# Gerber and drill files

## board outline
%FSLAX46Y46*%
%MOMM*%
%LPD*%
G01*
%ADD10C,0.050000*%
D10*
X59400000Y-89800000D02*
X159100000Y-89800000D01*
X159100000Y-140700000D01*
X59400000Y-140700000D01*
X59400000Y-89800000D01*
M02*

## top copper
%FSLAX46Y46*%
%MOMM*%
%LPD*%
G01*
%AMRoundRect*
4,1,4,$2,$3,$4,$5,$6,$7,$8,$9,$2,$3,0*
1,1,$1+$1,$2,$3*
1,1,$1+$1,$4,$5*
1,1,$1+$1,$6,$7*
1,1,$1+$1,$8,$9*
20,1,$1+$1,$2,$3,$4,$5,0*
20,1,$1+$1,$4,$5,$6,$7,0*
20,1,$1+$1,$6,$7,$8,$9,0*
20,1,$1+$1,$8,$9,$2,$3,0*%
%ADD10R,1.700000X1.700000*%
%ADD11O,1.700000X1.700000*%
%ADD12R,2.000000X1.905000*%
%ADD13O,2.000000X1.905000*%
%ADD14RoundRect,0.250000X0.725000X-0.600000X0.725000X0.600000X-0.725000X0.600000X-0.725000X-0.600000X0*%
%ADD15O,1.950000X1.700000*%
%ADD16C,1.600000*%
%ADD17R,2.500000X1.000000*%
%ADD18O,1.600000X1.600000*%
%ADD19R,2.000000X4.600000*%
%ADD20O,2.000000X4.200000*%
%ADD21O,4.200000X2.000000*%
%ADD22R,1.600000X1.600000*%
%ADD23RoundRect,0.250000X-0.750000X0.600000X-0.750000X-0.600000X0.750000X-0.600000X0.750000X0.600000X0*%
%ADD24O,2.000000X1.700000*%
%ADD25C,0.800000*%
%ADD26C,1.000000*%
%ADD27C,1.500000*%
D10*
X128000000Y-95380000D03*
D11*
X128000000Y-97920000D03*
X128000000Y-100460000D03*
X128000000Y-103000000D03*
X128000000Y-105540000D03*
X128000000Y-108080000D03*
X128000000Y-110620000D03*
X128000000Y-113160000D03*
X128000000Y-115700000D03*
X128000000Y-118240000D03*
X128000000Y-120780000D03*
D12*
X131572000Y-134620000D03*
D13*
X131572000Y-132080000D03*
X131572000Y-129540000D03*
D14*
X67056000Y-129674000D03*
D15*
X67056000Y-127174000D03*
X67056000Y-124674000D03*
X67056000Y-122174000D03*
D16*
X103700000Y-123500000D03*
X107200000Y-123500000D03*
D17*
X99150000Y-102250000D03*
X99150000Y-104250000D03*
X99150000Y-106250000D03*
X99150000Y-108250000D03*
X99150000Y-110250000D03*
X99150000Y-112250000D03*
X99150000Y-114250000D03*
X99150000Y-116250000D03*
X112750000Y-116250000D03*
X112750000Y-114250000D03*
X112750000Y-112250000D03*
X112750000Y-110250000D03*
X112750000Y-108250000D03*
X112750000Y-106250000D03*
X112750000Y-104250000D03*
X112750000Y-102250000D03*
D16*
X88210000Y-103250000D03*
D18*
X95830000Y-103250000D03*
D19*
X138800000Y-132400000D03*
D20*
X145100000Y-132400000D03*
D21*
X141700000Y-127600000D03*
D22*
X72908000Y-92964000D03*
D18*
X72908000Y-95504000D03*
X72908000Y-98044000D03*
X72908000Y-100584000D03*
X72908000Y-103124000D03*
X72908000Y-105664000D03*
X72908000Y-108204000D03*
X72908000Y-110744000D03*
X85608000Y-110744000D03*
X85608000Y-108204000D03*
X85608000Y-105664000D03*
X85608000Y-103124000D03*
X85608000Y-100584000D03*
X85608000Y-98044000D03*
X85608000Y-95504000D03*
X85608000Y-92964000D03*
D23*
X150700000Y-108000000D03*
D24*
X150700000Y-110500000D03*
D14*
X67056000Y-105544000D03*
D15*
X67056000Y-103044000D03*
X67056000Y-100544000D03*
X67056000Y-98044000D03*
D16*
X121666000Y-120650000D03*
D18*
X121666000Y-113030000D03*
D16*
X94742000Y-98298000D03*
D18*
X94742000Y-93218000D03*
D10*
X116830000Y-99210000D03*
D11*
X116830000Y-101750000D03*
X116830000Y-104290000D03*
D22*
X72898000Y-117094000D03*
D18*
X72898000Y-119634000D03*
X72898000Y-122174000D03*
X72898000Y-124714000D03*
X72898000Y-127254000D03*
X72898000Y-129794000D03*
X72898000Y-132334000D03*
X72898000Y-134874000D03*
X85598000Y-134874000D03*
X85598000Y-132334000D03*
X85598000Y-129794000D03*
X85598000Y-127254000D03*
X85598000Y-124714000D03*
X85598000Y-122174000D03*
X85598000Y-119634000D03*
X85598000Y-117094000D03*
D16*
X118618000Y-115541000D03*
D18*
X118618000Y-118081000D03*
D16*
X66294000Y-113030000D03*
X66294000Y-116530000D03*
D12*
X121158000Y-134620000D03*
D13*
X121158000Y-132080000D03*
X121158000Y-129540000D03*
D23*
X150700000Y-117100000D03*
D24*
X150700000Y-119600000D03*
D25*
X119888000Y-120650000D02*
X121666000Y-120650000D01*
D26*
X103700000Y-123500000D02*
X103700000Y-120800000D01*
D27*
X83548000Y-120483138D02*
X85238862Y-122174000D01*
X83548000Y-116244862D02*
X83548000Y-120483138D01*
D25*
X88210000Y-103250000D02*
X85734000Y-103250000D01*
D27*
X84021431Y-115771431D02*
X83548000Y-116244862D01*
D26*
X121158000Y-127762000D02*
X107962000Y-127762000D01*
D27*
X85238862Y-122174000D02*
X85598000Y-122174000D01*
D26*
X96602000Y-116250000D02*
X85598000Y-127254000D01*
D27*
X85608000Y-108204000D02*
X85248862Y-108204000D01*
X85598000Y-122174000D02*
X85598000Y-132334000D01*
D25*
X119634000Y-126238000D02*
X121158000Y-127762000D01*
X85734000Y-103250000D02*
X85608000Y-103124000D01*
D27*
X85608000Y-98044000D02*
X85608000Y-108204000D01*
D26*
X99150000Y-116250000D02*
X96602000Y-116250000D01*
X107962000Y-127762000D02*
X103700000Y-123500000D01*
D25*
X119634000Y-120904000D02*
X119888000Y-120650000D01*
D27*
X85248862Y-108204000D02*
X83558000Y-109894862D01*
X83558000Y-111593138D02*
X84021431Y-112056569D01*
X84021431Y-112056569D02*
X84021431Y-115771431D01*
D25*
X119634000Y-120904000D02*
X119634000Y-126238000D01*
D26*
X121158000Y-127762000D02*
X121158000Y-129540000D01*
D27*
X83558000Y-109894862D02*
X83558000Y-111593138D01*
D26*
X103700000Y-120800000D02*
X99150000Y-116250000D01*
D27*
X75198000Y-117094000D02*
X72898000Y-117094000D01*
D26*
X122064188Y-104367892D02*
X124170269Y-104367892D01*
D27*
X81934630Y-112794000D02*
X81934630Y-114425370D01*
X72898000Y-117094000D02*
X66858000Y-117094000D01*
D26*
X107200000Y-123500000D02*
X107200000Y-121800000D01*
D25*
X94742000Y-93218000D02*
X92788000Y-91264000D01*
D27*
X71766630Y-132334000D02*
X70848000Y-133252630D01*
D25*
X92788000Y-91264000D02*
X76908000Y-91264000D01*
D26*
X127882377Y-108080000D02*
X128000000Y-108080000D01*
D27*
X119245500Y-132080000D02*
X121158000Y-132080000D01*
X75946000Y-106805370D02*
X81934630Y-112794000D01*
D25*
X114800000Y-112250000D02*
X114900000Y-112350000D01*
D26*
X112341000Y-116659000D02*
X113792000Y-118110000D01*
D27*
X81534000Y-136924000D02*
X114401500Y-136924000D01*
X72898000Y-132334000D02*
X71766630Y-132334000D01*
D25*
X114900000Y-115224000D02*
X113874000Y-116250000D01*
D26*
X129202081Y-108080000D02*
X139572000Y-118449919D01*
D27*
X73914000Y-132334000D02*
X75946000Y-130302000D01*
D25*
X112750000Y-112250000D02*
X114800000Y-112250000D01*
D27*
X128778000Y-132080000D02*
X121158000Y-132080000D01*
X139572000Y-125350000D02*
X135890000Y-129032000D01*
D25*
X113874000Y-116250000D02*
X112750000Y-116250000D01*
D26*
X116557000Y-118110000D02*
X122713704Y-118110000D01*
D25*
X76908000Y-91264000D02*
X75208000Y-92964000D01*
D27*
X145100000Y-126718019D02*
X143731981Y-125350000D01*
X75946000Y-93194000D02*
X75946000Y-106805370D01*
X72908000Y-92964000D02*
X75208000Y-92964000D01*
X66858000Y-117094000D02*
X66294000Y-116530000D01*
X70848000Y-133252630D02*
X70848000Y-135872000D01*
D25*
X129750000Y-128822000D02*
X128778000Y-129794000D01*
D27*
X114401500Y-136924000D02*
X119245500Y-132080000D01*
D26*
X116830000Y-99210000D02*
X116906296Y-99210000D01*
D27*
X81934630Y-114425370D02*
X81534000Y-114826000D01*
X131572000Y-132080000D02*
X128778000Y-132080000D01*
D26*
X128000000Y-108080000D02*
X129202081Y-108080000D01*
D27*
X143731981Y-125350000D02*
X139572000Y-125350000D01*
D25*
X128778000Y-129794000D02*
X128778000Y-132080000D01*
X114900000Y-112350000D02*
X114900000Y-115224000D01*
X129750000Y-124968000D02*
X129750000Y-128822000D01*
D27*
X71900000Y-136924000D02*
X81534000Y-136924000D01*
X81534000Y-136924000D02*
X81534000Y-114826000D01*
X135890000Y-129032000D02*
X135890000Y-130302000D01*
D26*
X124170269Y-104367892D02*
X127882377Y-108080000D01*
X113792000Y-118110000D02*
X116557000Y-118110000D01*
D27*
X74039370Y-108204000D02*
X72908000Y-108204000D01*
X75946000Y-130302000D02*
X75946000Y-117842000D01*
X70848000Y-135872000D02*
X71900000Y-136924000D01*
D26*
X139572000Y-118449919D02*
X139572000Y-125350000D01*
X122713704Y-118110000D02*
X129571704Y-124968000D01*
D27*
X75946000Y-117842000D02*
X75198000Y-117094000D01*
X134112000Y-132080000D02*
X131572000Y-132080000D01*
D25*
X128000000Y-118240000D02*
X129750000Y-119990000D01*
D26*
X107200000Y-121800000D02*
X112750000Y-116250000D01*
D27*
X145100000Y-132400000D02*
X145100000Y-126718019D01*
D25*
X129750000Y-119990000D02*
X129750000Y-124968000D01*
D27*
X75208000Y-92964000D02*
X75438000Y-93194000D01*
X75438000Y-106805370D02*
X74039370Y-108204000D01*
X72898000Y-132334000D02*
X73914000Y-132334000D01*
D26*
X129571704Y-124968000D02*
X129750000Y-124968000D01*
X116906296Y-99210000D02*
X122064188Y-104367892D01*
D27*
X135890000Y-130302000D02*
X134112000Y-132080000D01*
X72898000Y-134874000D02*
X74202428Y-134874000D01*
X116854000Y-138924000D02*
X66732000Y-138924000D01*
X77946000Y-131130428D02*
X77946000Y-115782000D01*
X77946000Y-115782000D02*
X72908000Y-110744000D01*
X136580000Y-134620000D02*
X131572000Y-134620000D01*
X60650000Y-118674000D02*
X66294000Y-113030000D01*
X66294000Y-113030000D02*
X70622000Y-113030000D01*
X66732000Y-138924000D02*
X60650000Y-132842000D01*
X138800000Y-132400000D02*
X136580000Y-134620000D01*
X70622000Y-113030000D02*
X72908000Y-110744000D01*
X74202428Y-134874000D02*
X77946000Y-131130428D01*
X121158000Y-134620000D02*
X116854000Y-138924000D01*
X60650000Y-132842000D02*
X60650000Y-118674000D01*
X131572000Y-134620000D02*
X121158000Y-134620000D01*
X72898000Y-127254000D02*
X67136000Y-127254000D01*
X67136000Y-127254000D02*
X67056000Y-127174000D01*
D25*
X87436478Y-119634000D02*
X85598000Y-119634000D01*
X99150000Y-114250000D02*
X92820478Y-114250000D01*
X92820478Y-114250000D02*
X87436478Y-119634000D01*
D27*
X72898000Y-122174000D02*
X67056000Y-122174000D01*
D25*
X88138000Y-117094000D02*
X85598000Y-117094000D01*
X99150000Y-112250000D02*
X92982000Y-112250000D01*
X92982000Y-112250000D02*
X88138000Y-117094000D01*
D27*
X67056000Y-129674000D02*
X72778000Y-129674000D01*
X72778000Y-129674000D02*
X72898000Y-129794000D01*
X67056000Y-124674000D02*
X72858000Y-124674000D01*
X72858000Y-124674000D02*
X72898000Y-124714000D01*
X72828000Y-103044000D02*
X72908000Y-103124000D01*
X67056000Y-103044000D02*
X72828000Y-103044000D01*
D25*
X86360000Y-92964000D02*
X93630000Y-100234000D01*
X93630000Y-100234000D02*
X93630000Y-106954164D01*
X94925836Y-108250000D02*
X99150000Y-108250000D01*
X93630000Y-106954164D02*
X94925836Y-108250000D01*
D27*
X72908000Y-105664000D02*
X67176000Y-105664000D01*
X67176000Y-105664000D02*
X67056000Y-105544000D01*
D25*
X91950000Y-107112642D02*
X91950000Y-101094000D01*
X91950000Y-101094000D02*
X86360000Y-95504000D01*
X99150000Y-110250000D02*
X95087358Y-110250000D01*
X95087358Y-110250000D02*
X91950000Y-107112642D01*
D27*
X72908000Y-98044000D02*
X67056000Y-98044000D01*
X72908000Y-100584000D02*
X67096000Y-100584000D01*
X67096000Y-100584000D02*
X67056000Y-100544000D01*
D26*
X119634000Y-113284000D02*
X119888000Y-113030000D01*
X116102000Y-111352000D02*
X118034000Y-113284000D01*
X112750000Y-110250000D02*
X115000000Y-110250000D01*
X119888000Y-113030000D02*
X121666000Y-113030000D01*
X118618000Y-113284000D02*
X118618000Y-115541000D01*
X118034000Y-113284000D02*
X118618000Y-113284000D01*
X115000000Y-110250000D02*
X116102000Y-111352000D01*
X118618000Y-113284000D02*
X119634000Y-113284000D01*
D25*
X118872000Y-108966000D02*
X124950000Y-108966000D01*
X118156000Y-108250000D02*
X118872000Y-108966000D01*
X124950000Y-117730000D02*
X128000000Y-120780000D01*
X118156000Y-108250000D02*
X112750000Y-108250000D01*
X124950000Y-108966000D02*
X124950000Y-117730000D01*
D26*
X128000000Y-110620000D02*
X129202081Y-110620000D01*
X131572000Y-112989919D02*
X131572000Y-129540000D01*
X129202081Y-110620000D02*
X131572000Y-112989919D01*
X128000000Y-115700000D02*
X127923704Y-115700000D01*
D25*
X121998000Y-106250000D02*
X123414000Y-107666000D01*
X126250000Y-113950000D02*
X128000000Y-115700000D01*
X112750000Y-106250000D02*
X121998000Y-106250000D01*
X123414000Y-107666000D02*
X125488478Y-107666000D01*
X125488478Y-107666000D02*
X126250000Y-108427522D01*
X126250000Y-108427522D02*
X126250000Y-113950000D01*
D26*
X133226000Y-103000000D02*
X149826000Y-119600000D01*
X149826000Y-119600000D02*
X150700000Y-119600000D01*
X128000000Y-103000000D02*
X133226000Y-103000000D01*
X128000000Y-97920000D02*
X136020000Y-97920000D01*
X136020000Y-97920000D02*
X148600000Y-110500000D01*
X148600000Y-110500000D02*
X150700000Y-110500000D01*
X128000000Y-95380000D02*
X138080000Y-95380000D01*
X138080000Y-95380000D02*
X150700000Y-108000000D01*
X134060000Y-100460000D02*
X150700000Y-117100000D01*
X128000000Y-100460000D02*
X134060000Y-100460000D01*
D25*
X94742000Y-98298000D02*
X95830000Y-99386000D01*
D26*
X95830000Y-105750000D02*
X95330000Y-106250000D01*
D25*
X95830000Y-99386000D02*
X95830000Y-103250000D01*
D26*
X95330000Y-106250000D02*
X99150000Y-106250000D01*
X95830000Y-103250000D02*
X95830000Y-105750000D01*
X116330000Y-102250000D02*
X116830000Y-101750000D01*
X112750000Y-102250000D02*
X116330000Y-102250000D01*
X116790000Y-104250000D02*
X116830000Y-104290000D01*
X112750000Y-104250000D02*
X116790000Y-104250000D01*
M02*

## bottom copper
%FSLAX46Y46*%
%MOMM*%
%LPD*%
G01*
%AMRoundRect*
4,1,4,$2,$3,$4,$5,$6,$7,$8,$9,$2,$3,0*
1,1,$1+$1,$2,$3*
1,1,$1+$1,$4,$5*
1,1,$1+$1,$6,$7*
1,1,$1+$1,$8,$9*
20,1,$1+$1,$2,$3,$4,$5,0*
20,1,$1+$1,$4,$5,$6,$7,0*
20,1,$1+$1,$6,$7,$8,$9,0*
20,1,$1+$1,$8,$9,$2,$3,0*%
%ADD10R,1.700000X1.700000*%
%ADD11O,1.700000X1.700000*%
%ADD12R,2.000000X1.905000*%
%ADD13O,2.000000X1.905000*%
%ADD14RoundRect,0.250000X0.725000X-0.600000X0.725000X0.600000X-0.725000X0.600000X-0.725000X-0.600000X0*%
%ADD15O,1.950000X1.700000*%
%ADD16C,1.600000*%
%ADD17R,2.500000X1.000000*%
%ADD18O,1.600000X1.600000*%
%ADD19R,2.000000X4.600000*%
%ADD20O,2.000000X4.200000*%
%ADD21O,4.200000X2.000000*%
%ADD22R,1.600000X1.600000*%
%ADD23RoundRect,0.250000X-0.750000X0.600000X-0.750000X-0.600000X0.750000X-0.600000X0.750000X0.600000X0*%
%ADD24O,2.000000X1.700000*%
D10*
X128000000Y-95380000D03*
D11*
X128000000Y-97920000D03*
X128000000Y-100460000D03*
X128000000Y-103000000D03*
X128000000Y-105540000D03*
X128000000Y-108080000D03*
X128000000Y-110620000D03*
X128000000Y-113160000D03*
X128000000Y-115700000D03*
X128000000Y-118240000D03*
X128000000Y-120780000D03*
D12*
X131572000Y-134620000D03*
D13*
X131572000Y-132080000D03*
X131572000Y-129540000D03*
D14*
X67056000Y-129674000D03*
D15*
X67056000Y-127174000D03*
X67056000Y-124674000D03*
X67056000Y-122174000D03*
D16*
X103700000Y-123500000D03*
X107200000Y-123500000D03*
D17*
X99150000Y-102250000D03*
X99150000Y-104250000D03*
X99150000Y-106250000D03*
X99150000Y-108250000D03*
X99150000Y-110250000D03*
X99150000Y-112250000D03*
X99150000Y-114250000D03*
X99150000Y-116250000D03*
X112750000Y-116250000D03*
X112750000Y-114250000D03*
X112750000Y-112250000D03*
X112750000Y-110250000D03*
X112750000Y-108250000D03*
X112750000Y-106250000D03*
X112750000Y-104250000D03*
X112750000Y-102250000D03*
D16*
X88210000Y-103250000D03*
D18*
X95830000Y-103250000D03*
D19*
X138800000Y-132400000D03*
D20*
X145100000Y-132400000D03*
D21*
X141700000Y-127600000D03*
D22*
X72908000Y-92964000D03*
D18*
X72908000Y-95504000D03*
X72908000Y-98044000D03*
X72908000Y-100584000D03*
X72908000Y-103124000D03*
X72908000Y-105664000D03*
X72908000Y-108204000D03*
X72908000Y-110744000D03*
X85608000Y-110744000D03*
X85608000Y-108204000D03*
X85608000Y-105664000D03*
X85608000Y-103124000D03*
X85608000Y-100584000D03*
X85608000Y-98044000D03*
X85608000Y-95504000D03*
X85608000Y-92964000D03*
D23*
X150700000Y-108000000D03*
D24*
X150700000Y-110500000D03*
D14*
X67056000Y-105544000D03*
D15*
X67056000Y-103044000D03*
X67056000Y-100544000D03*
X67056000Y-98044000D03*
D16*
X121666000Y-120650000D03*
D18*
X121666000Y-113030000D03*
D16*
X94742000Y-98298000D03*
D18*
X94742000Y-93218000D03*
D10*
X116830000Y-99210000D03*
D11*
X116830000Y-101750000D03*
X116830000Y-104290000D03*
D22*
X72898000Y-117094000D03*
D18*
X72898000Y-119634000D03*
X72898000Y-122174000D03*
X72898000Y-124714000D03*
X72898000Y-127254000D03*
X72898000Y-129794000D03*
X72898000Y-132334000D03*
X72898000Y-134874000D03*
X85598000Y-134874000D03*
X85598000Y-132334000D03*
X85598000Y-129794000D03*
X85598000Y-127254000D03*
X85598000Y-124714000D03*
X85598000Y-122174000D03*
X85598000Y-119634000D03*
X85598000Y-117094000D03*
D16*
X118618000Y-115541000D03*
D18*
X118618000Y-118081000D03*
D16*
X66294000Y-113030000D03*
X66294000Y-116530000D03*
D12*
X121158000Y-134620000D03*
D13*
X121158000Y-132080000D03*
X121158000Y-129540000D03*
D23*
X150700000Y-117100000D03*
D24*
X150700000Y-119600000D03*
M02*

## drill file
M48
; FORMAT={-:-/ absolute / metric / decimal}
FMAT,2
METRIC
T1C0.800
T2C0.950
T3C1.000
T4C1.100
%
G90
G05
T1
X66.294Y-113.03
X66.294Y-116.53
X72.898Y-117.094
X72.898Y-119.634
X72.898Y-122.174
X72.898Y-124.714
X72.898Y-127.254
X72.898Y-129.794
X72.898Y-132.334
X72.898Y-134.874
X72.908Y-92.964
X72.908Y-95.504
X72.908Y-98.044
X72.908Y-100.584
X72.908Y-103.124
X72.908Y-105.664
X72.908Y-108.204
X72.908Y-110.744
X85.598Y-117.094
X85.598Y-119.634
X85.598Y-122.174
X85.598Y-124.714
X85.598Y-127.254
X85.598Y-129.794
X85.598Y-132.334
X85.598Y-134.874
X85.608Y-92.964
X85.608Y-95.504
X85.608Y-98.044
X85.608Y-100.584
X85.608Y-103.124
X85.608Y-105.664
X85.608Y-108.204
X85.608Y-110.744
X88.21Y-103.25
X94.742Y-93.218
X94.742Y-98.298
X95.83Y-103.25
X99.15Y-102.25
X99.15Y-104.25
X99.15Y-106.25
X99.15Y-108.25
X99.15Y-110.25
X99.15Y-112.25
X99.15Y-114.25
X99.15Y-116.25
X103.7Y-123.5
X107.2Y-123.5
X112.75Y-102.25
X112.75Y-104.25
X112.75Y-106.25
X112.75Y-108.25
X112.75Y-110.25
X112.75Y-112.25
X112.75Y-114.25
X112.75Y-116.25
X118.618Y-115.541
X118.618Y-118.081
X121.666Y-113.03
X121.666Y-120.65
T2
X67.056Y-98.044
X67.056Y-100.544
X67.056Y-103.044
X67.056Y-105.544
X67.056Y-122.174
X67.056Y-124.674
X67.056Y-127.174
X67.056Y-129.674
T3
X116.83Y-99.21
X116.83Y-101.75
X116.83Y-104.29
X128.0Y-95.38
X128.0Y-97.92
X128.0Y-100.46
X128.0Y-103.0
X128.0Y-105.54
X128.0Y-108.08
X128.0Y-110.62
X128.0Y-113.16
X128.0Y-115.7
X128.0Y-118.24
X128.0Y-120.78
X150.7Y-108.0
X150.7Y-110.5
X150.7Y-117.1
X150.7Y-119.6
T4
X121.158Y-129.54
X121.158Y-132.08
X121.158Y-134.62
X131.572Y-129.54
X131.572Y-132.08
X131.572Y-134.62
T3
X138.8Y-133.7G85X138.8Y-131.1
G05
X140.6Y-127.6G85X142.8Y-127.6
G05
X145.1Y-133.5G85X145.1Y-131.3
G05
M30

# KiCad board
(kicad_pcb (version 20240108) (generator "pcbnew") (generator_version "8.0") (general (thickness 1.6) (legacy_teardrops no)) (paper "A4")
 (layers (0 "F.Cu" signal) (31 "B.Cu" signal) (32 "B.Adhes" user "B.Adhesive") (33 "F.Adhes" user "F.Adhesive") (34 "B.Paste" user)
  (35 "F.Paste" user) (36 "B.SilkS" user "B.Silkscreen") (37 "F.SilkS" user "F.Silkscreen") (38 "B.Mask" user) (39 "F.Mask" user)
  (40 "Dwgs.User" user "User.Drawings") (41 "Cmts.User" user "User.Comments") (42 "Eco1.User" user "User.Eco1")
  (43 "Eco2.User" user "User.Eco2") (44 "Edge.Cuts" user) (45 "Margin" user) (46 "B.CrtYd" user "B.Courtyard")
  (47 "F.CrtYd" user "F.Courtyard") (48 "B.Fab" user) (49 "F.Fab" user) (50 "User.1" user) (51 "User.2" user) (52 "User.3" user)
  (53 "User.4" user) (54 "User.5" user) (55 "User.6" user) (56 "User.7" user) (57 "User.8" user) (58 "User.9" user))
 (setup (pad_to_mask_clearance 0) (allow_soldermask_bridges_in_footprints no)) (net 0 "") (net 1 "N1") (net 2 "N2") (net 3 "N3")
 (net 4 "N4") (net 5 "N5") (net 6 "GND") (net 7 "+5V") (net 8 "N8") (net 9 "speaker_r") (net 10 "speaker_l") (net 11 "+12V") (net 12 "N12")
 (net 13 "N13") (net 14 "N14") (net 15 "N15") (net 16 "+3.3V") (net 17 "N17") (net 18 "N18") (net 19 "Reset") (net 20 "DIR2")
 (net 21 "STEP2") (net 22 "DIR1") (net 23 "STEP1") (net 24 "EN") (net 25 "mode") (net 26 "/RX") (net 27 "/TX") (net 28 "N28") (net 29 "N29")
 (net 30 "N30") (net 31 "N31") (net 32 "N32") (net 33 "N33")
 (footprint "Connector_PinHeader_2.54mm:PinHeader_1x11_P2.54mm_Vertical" (layer "F.Cu") (at 128 95.38)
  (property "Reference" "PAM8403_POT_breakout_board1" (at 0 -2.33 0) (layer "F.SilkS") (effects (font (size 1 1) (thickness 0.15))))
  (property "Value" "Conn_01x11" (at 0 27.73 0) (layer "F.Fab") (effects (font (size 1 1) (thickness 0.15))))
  (pad "1" thru_hole rect (at 0 0) (size 1.7 1.7) (drill 1) (layers "*.Cu" "*.Mask") (remove_unused_layers no) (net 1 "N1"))
  (pad "2" thru_hole oval (at 0 2.54) (size 1.7 1.7) (drill 1) (layers "*.Cu" "*.Mask") (remove_unused_layers no) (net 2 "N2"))
  (pad "3" thru_hole oval (at 0 5.08) (size 1.7 1.7) (drill 1) (layers "*.Cu" "*.Mask") (remove_unused_layers no) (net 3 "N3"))
  (pad "4" thru_hole oval (at 0 7.62) (size 1.7 1.7) (drill 1) (layers "*.Cu" "*.Mask") (remove_unused_layers no) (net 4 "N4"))
  (pad "5" thru_hole oval (at 0 10.16) (size 1.7 1.7) (drill 1) (layers "*.Cu" "*.Mask") (remove_unused_layers no) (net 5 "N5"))
  (pad "6" thru_hole oval (at 0 12.7) (size 1.7 1.7) (drill 1) (layers "*.Cu" "*.Mask") (remove_unused_layers no) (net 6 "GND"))
  (pad "7" thru_hole oval (at 0 15.24) (size 1.7 1.7) (drill 1) (layers "*.Cu" "*.Mask") (remove_unused_layers no) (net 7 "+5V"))
  (pad "8" thru_hole oval (at 0 17.78) (size 1.7 1.7) (drill 1) (layers "*.Cu" "*.Mask") (remove_unused_layers no) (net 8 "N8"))
  (pad "9" thru_hole oval (at 0 20.32) (size 1.7 1.7) (drill 1) (layers "*.Cu" "*.Mask") (remove_unused_layers no) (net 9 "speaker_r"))
  (pad "10" thru_hole oval (at 0 22.86) (size 1.7 1.7) (drill 1) (layers "*.Cu" "*.Mask") (remove_unused_layers no) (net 6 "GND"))
  (pad "11" thru_hole oval (at 0 25.4) (size 1.7 1.7) (drill 1) (layers "*.Cu" "*.Mask") (remove_unused_layers no) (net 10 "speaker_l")))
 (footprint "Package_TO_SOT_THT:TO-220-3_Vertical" (layer "F.Cu") (at 131.572 134.62 90)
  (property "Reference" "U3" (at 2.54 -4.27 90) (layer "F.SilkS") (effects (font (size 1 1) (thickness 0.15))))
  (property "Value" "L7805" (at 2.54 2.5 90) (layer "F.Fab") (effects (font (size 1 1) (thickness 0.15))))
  (pad "1" thru_hole rect (at 0 0 90) (size 1.905 2) (drill 1.1) (layers "*.Cu" "*.Mask") (remove_unused_layers no) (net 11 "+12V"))
  (pad "2" thru_hole oval (at 2.54 0 90) (size 1.905 2) (drill 1.1) (layers "*.Cu" "*.Mask") (remove_unused_layers no) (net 6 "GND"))
  (pad "3" thru_hole oval (at 5.08 0 90) (size 1.905 2) (drill 1.1) (layers "*.Cu" "*.Mask") (remove_unused_layers no) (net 7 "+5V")))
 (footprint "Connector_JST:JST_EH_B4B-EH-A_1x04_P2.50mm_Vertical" (layer "F.Cu") (at 67.056 129.674 90)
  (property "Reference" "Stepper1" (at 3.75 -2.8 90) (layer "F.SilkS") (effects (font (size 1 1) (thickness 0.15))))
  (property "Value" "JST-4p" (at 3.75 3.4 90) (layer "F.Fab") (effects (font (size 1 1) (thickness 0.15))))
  (pad "1" thru_hole roundrect (at 0 0 90) (size 1.7 1.95) (drill 0.95) (layers "*.Cu" "*.Mask") (remove_unused_layers no)
   (roundrect_rratio 0.147059) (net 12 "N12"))
  (pad "2" thru_hole oval (at 2.5 0 90) (size 1.7 1.95) (drill 0.95) (layers "*.Cu" "*.Mask") (remove_unused_layers no) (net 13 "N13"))
  (pad "3" thru_hole oval (at 5 0 90) (size 1.7 1.95) (drill 0.95) (layers "*.Cu" "*.Mask") (remove_unused_layers no) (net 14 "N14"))
  (pad "4" thru_hole oval (at 7.5 0 90) (size 1.7 1.95) (drill 0.95) (layers "*.Cu" "*.Mask") (remove_unused_layers no) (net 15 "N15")))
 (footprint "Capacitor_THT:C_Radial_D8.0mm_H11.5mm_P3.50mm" (layer "F.Cu") (at 103.7 123.5)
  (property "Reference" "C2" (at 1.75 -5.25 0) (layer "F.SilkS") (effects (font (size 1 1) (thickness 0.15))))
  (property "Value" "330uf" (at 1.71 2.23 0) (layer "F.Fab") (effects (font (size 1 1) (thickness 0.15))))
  (pad "1" thru_hole circle (at 0 0) (size 1.6 1.6) (drill 0.8) (layers "*.Cu" "*.Mask") (remove_unused_layers no) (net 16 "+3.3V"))
  (pad "2" thru_hole circle (at 3.5 0) (size 1.6 1.6) (drill 0.8) (layers "*.Cu" "*.Mask") (remove_unused_layers no) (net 6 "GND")))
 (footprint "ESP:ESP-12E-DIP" (layer "F.Cu") (at 105.95 106.45)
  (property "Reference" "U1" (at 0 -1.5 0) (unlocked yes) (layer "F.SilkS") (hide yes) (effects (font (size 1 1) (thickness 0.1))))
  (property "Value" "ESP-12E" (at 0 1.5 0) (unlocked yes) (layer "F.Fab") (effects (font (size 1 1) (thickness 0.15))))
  (pad "1" thru_hole rect (at -6.8 -4.2) (size 2.5 1) (drill 0.8) (layers "*.Cu" "*.Mask") (remove_unused_layers no) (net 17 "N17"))
  (pad "2" thru_hole rect (at -6.8 -2.2) (size 2.5 1) (drill 0.8) (layers "*.Cu" "*.Mask") (remove_unused_layers no) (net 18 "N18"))
  (pad "3" thru_hole rect (at -6.8 -0.2) (size 2.5 1) (drill 0.8) (layers "*.Cu" "*.Mask") (remove_unused_layers no) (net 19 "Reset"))
  (pad "4" thru_hole rect (at -6.8 1.8) (size 2.5 1) (drill 0.8) (layers "*.Cu" "*.Mask") (remove_unused_layers no) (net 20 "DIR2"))
  (pad "5" thru_hole rect (at -6.8 3.8) (size 2.5 1) (drill 0.8) (layers "*.Cu" "*.Mask") (remove_unused_layers no) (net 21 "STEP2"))
  (pad "6" thru_hole rect (at -6.8 5.8) (size 2.5 1) (drill 0.8) (layers "*.Cu" "*.Mask") (remove_unused_layers no) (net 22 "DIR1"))
  (pad "7" thru_hole rect (at -6.8 7.8) (size 2.5 1) (drill 0.8) (layers "*.Cu" "*.Mask") (remove_unused_layers no) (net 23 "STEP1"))
  (pad "8" thru_hole rect (at -6.8 9.8) (size 2.5 1) (drill 0.8) (layers "*.Cu" "*.Mask") (remove_unused_layers no) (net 16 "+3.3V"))
  (pad "15" thru_hole rect (at 6.8 9.8) (size 2.5 1) (drill 0.8) (layers "*.Cu" "*.Mask") (remove_unused_layers no) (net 6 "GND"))
  (pad "16" thru_hole rect (at 6.8 7.8) (size 2.5 1) (drill 0.8) (layers "*.Cu" "*.Mask") (remove_unused_layers no) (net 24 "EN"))
  (pad "17" thru_hole rect (at 6.8 5.8) (size 2.5 1) (drill 0.8) (layers "*.Cu" "*.Mask") (remove_unused_layers no) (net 6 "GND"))
  (pad "18" thru_hole rect (at 6.8 3.8) (size 2.5 1) (drill 0.8) (layers "*.Cu" "*.Mask") (remove_unused_layers no) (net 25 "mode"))
  (pad "19" thru_hole rect (at 6.8 1.8) (size 2.5 1) (drill 0.8) (layers "*.Cu" "*.Mask") (remove_unused_layers no) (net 10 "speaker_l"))
  (pad "20" thru_hole rect (at 6.8 -0.2) (size 2.5 1) (drill 0.8) (layers "*.Cu" "*.Mask") (remove_unused_layers no) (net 9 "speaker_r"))
  (pad "21" thru_hole rect (at 6.8 -2.2) (size 2.5 1) (drill 0.8) (layers "*.Cu" "*.Mask") (remove_unused_layers no) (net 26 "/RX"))
  (pad "22" thru_hole rect (at 6.8 -4.2) (size 2.5 1) (drill 0.8) (layers "*.Cu" "*.Mask") (remove_unused_layers no) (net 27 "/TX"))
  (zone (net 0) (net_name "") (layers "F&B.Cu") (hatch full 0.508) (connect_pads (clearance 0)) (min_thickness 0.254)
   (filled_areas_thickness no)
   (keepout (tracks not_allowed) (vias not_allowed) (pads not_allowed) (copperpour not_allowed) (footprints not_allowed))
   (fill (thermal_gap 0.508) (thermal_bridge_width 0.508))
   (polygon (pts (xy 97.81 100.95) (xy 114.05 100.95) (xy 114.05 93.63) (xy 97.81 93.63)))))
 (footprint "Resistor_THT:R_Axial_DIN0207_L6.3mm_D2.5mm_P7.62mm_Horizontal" (layer "F.Cu") (at 88.21 103.25)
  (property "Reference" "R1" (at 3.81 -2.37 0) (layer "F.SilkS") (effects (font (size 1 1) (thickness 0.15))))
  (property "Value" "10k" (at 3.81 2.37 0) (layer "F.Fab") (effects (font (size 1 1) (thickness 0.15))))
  (pad "1" thru_hole circle (at 0 0) (size 1.6 1.6) (drill 0.8) (layers "*.Cu" "*.Mask") (remove_unused_layers no) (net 16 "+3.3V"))
  (pad "2" thru_hole oval (at 7.62 0) (size 1.6 1.6) (drill 0.8) (layers "*.Cu" "*.Mask") (remove_unused_layers no) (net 19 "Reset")))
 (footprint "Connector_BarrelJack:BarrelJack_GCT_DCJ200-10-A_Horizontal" (layer "F.Cu") (at 138.8 132.4 90)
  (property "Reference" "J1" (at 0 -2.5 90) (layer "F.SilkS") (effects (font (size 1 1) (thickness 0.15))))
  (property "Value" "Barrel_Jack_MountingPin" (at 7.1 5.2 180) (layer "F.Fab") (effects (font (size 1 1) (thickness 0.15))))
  (pad "1" thru_hole rect (at 0 0 90) (size 4.6 2) (drill oval 3.6 1) (layers "*.Cu" "*.Mask") (remove_unused_layers no) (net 11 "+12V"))
  (pad "2" thru_hole oval (at 0 6.3 90) (size 4.2 2) (drill oval 3.2 1) (layers "*.Cu" "*.Mask") (remove_unused_layers no) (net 6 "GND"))
  (pad "3" thru_hole oval (at 4.8 2.9 90) (size 2 4.2) (drill oval 1 3.2) (layers "*.Cu" "*.Mask") (remove_unused_layers no)))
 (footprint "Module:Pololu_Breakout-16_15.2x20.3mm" (layer "F.Cu") (at 72.908 92.964)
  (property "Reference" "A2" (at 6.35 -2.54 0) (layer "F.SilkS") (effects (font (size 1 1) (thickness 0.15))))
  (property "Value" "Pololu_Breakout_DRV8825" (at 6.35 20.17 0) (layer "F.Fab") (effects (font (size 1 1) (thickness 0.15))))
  (pad "1" thru_hole rect (at 0 0) (size 1.6 1.6) (drill 0.8) (layers "*.Cu" "*.Mask") (remove_unused_layers no) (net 6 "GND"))
  (pad "2" thru_hole oval (at 0 2.54) (size 1.6 1.6) (drill 0.8) (layers "*.Cu" "*.Mask") (remove_unused_layers no) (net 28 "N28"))
  (pad "3" thru_hole oval (at 0 5.08) (size 1.6 1.6) (drill 0.8) (layers "*.Cu" "*.Mask") (remove_unused_layers no) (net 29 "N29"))
  (pad "4" thru_hole oval (at 0 7.62) (size 1.6 1.6) (drill 0.8) (layers "*.Cu" "*.Mask") (remove_unused_layers no) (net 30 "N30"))
  (pad "5" thru_hole oval (at 0 10.16) (size 1.6 1.6) (drill 0.8) (layers "*.Cu" "*.Mask") (remove_unused_layers no) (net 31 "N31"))
  (pad "6" thru_hole oval (at 0 12.7) (size 1.6 1.6) (drill 0.8) (layers "*.Cu" "*.Mask") (remove_unused_layers no) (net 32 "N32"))
  (pad "7" thru_hole oval (at 0 15.24) (size 1.6 1.6) (drill 0.8) (layers "*.Cu" "*.Mask") (remove_unused_layers no) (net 6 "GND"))
  (pad "8" thru_hole oval (at 0 17.78) (size 1.6 1.6) (drill 0.8) (layers "*.Cu" "*.Mask") (remove_unused_layers no) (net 11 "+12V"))
  (pad "9" thru_hole oval (at 12.7 17.78) (size 1.6 1.6) (drill 0.8) (layers "*.Cu" "*.Mask") (remove_unused_layers no) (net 24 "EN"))
  (pad "10" thru_hole oval (at 12.7 15.24) (size 1.6 1.6) (drill 0.8) (layers "*.Cu" "*.Mask") (remove_unused_layers no) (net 16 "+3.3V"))
  (pad "11" thru_hole oval (at 12.7 12.7) (size 1.6 1.6) (drill 0.8) (layers "*.Cu" "*.Mask") (remove_unused_layers no) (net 16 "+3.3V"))
  (pad "12" thru_hole oval (at 12.7 10.16) (size 1.6 1.6) (drill 0.8) (layers "*.Cu" "*.Mask") (remove_unused_layers no) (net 16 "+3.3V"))
  (pad "13" thru_hole oval (at 12.7 7.62) (size 1.6 1.6) (drill 0.8) (layers "*.Cu" "*.Mask") (remove_unused_layers no) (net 16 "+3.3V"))
  (pad "14" thru_hole oval (at 12.7 5.08) (size 1.6 1.6) (drill 0.8) (layers "*.Cu" "*.Mask") (remove_unused_layers no) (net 16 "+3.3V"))
  (pad "15" thru_hole oval (at 12.7 2.54) (size 1.6 1.6) (drill 0.8) (layers "*.Cu" "*.Mask") (remove_unused_layers no) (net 21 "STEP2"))
  (pad "16" thru_hole oval (at 12.7 0) (size 1.6 1.6) (drill 0.8) (layers "*.Cu" "*.Mask") (remove_unused_layers no) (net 20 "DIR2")))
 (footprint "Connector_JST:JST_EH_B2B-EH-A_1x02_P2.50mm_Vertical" (layer "F.Cu") (at 150.7 108 -90)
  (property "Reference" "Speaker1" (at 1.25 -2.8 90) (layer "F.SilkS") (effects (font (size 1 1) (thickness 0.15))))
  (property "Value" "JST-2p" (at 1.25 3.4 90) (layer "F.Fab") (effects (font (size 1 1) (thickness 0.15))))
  (pad "1" thru_hole roundrect (at 0 0 270) (size 1.7 2) (drill 1) (layers "*.Cu" "*.Mask") (remove_unused_layers no)
   (roundrect_rratio 0.147059) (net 1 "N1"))
  (pad "2" thru_hole oval (at 2.5 0 270) (size 1.7 2) (drill 1) (layers "*.Cu" "*.Mask") (remove_unused_layers no) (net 2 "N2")))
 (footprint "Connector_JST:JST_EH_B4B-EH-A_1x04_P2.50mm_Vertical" (layer "F.Cu") (at 67.056 105.544 90)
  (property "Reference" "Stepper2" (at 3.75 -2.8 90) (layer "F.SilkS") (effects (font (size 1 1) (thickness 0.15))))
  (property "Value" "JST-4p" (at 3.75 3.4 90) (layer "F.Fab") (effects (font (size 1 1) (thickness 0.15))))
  (pad "1" thru_hole roundrect (at 0 0 90) (size 1.7 1.95) (drill 0.95) (layers "*.Cu" "*.Mask") (remove_unused_layers no)
   (roundrect_rratio 0.147059) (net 32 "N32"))
  (pad "2" thru_hole oval (at 2.5 0 90) (size 1.7 1.95) (drill 0.95) (layers "*.Cu" "*.Mask") (remove_unused_layers no) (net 31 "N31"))
  (pad "3" thru_hole oval (at 5 0 90) (size 1.7 1.95) (drill 0.95) (layers "*.Cu" "*.Mask") (remove_unused_layers no) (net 30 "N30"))
  (pad "4" thru_hole oval (at 7.5 0 90) (size 1.7 1.95) (drill 0.95) (layers "*.Cu" "*.Mask") (remove_unused_layers no) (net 29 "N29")))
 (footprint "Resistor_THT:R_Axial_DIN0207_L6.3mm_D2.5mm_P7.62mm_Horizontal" (layer "F.Cu") (at 121.666 120.65 90)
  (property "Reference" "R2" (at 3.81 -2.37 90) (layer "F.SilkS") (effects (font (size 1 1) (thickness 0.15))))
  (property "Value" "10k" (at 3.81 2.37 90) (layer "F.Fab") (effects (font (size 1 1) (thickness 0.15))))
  (pad "1" thru_hole circle (at 0 0 90) (size 1.6 1.6) (drill 0.8) (layers "*.Cu" "*.Mask") (remove_unused_layers no) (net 16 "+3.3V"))
  (pad "2" thru_hole oval (at 7.62 0 90) (size 1.6 1.6) (drill 0.8) (layers "*.Cu" "*.Mask") (remove_unused_layers no) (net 25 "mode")))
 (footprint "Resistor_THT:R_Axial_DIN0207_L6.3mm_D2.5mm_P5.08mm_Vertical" (layer "F.Cu") (at 94.742 98.298 90)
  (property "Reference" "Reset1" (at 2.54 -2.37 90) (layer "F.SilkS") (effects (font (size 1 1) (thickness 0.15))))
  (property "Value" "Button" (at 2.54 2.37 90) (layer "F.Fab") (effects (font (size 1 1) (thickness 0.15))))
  (pad "1" thru_hole circle (at 0 0 90) (size 1.6 1.6) (drill 0.8) (layers "*.Cu" "*.Mask") (remove_unused_layers no) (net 19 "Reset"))
  (pad "2" thru_hole oval (at 5.08 0 90) (size 1.6 1.6) (drill 0.8) (layers "*.Cu" "*.Mask") (remove_unused_layers no) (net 6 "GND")))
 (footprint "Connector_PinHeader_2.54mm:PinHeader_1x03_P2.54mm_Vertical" (layer "F.Cu") (at 116.83 99.21)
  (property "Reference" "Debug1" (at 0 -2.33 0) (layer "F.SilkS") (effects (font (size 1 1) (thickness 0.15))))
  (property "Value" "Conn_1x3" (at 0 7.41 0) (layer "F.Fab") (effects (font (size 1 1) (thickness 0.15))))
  (pad "1" thru_hole rect (at 0 0) (size 1.7 1.7) (drill 1) (layers "*.Cu" "*.Mask") (remove_unused_layers no) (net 6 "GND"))
  (pad "2" thru_hole oval (at 0 2.54) (size 1.7 1.7) (drill 1) (layers "*.Cu" "*.Mask") (remove_unused_layers no) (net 27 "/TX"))
  (pad "3" thru_hole oval (at 0 5.08) (size 1.7 1.7) (drill 1) (layers "*.Cu" "*.Mask") (remove_unused_layers no) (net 26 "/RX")))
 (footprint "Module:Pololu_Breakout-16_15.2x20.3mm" (layer "F.Cu") (at 72.898 117.094)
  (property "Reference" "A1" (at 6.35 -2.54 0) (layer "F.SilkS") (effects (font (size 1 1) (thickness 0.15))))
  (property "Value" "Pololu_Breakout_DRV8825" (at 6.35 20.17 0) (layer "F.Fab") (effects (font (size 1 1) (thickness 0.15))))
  (pad "1" thru_hole rect (at 0 0) (size 1.6 1.6) (drill 0.8) (layers "*.Cu" "*.Mask") (remove_unused_layers no) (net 6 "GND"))
  (pad "2" thru_hole oval (at 0 2.54) (size 1.6 1.6) (drill 0.8) (layers "*.Cu" "*.Mask") (remove_unused_layers no) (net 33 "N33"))
  (pad "3" thru_hole oval (at 0 5.08) (size 1.6 1.6) (drill 0.8) (layers "*.Cu" "*.Mask") (remove_unused_layers no) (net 15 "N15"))
  (pad "4" thru_hole oval (at 0 7.62) (size 1.6 1.6) (drill 0.8) (layers "*.Cu" "*.Mask") (remove_unused_layers no) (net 14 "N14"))
  (pad "5" thru_hole oval (at 0 10.16) (size 1.6 1.6) (drill 0.8) (layers "*.Cu" "*.Mask") (remove_unused_layers no) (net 13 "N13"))
  (pad "6" thru_hole oval (at 0 12.7) (size 1.6 1.6) (drill 0.8) (layers "*.Cu" "*.Mask") (remove_unused_layers no) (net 12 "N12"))
  (pad "7" thru_hole oval (at 0 15.24) (size 1.6 1.6) (drill 0.8) (layers "*.Cu" "*.Mask") (remove_unused_layers no) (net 6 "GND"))
  (pad "8" thru_hole oval (at 0 17.78) (size 1.6 1.6) (drill 0.8) (layers "*.Cu" "*.Mask") (remove_unused_layers no) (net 11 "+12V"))
  (pad "9" thru_hole oval (at 12.7 17.78) (size 1.6 1.6) (drill 0.8) (layers "*.Cu" "*.Mask") (remove_unused_layers no) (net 24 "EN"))
  (pad "10" thru_hole oval (at 12.7 15.24) (size 1.6 1.6) (drill 0.8) (layers "*.Cu" "*.Mask") (remove_unused_layers no) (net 16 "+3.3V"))
  (pad "11" thru_hole oval (at 12.7 12.7) (size 1.6 1.6) (drill 0.8) (layers "*.Cu" "*.Mask") (remove_unused_layers no) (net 16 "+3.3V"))
  (pad "12" thru_hole oval (at 12.7 10.16) (size 1.6 1.6) (drill 0.8) (layers "*.Cu" "*.Mask") (remove_unused_layers no) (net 16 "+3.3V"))
  (pad "13" thru_hole oval (at 12.7 7.62) (size 1.6 1.6) (drill 0.8) (layers "*.Cu" "*.Mask") (remove_unused_layers no) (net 16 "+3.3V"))
  (pad "14" thru_hole oval (at 12.7 5.08) (size 1.6 1.6) (drill 0.8) (layers "*.Cu" "*.Mask") (remove_unused_layers no) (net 16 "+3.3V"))
  (pad "15" thru_hole oval (at 12.7 2.54) (size 1.6 1.6) (drill 0.8) (layers "*.Cu" "*.Mask") (remove_unused_layers no) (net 23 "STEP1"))
  (pad "16" thru_hole oval (at 12.7 0) (size 1.6 1.6) (drill 0.8) (layers "*.Cu" "*.Mask") (remove_unused_layers no) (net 22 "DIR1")))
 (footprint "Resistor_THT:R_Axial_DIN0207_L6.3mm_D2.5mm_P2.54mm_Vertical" (layer "F.Cu") (at 118.618 115.541 -90)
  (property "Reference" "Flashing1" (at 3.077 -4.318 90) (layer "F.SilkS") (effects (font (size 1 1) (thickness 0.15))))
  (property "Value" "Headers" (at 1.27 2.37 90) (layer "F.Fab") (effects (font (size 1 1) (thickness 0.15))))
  (pad "1" thru_hole circle (at 0 0 270) (size 1.6 1.6) (drill 0.8) (layers "*.Cu" "*.Mask") (remove_unused_layers no) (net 25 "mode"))
  (pad "2" thru_hole oval (at 2.54 0 270) (size 1.6 1.6) (drill 0.8) (layers "*.Cu" "*.Mask") (remove_unused_layers no) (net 6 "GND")))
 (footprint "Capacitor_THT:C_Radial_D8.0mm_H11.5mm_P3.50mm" (layer "F.Cu") (at 66.294 113.03 -90)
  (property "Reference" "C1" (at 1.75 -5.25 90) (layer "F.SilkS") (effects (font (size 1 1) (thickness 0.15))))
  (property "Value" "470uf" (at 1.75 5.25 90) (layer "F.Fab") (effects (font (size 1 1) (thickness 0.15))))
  (pad "1" thru_hole circle (at 0 0 270) (size 1.6 1.6) (drill 0.8) (layers "*.Cu" "*.Mask") (remove_unused_layers no) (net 11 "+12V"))
  (pad "2" thru_hole circle (at 3.5 0 270) (size 1.6 1.6) (drill 0.8) (layers "*.Cu" "*.Mask") (remove_unused_layers no) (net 6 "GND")))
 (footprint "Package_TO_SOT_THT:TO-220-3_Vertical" (layer "F.Cu") (at 121.158 134.62 90)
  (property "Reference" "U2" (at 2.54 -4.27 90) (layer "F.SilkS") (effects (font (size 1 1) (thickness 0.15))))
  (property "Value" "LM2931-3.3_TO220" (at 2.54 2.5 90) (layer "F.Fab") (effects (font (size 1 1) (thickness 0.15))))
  (pad "1" thru_hole rect (at 0 0 90) (size 1.905 2) (drill 1.1) (layers "*.Cu" "*.Mask") (remove_unused_layers no) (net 11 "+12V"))
  (pad "2" thru_hole oval (at 2.54 0 90) (size 1.905 2) (drill 1.1) (layers "*.Cu" "*.Mask") (remove_unused_layers no) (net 6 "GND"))
  (pad "3" thru_hole oval (at 5.08 0 90) (size 1.905 2) (drill 1.1) (layers "*.Cu" "*.Mask") (remove_unused_layers no) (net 16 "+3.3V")))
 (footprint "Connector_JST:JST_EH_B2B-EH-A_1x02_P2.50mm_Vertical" (layer "F.Cu") (at 150.7 117.1 -90)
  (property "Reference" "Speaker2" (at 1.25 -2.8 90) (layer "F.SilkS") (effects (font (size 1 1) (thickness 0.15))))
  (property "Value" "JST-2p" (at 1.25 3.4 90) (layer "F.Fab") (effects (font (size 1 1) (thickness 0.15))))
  (pad "1" thru_hole roundrect (at 0 0 270) (size 1.7 2) (drill 1) (layers "*.Cu" "*.Mask") (remove_unused_layers no)
   (roundrect_rratio 0.147059) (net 3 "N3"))
  (pad "2" thru_hole oval (at 2.5 0 270) (size 1.7 2) (drill 1) (layers "*.Cu" "*.Mask") (remove_unused_layers no) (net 4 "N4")))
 (gr_rect (start 59.4 89.8) (end 159.1 140.7) (stroke (width 0.05) (type default)) (fill none) (layer "Edge.Cuts"))
 (segment (start 119.888 120.65) (end 121.666 120.65) (width 0.8) (layer "F.Cu") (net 16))
 (segment (start 103.7 123.5) (end 103.7 120.8) (width 1) (layer "F.Cu") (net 16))
 (segment (start 83.548 120.483138) (end 85.238862 122.174) (width 1.5) (layer "F.Cu") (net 16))
 (segment (start 83.548 116.244862) (end 83.548 120.483138) (width 1.5) (layer "F.Cu") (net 16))
 (segment (start 88.21 103.25) (end 85.734 103.25) (width 0.8) (layer "F.Cu") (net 16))
 (segment (start 84.021431 115.771431) (end 83.548 116.244862) (width 1.5) (layer "F.Cu") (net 16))
 (segment (start 121.158 127.762) (end 107.962 127.762) (width 1) (layer "F.Cu") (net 16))
 (segment (start 85.238862 122.174) (end 85.598 122.174) (width 1.5) (layer "F.Cu") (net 16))
 (segment (start 96.602 116.25) (end 85.598 127.254) (width 1) (layer "F.Cu") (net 16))
 (segment (start 85.608 108.204) (end 85.248862 108.204) (width 1.5) (layer "F.Cu") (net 16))
 (segment (start 85.598 122.174) (end 85.598 132.334) (width 1.5) (layer "F.Cu") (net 16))
 (segment (start 119.634 126.238) (end 121.158 127.762) (width 0.8) (layer "F.Cu") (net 16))
 (segment (start 85.734 103.25) (end 85.608 103.124) (width 0.8) (layer "F.Cu") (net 16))
 (segment (start 85.608 98.044) (end 85.608 108.204) (width 1.5) (layer "F.Cu") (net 16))
 (segment (start 99.15 116.25) (end 96.602 116.25) (width 1) (layer "F.Cu") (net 16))
 (segment (start 107.962 127.762) (end 103.7 123.5) (width 1) (layer "F.Cu") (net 16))
 (segment (start 119.634 120.904) (end 119.888 120.65) (width 0.8) (layer "F.Cu") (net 16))
 (segment (start 85.248862 108.204) (end 83.558 109.894862) (width 1.5) (layer "F.Cu") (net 16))
 (segment (start 83.558 111.593138) (end 84.021431 112.056569) (width 1.5) (layer "F.Cu") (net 16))
 (segment (start 84.021431 112.056569) (end 84.021431 115.771431) (width 1.5) (layer "F.Cu") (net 16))
 (segment (start 119.634 120.904) (end 119.634 126.238) (width 0.8) (layer "F.Cu") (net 16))
 (segment (start 121.158 127.762) (end 121.158 129.54) (width 1) (layer "F.Cu") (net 16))
 (segment (start 83.558 109.894862) (end 83.558 111.593138) (width 1.5) (layer "F.Cu") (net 16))
 (segment (start 103.7 120.8) (end 99.15 116.25) (width 1) (layer "F.Cu") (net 16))
 (segment (start 75.198 117.094) (end 72.898 117.094) (width 1.5) (layer "F.Cu") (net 6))
 (segment (start 122.064188 104.367892) (end 124.170269 104.367892) (width 1) (layer "F.Cu") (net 6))
 (segment (start 81.93463 112.794) (end 81.93463 114.42537) (width 1.5) (layer "F.Cu") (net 6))
 (segment (start 72.898 117.094) (end 66.858 117.094) (width 1.5) (layer "F.Cu") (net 6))
 (segment (start 107.2 123.5) (end 107.2 121.8) (width 1) (layer "F.Cu") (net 6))
 (segment (start 94.742 93.218) (end 92.788 91.264) (width 0.8) (layer "F.Cu") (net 6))
 (segment (start 71.76663 132.334) (end 70.848 133.25263) (width 1.5) (layer "F.Cu") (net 6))
 (segment (start 92.788 91.264) (end 76.908 91.264) (width 0.8) (layer "F.Cu") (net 6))
 (segment (start 127.882377 108.08) (end 128 108.08) (width 1) (layer "F.Cu") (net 6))
 (segment (start 119.2455 132.08) (end 121.158 132.08) (width 1.5) (layer "F.Cu") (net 6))
 (segment (start 75.946 106.80537) (end 81.93463 112.794) (width 1.5) (layer "F.Cu") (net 6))
 (segment (start 114.8 112.25) (end 114.9 112.35) (width 0.8) (layer "F.Cu") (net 6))
 (segment (start 112.341 116.659) (end 113.792 118.11) (width 1) (layer "F.Cu") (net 6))
 (segment (start 81.534 136.924) (end 114.4015 136.924) (width 1.5) (layer "F.Cu") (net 6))
 (segment (start 72.898 132.334) (end 71.76663 132.334) (width 1.5) (layer "F.Cu") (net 6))
 (segment (start 114.9 115.224) (end 113.874 116.25) (width 0.8) (layer "F.Cu") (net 6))
 (segment (start 129.202081 108.08) (end 139.572 118.449919) (width 1) (layer "F.Cu") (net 6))
 (segment (start 73.914 132.334) (end 75.946 130.302) (width 1.5) (layer "F.Cu") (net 6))
 (segment (start 112.75 112.25) (end 114.8 112.25) (width 0.8) (layer "F.Cu") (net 6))
 (segment (start 128.778 132.08) (end 121.158 132.08) (width 1.5) (layer "F.Cu") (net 6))
 (segment (start 139.572 125.35) (end 135.89 129.032) (width 1.5) (layer "F.Cu") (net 6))
 (segment (start 113.874 116.25) (end 112.75 116.25) (width 0.8) (layer "F.Cu") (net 6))
 (segment (start 116.557 118.11) (end 122.713704 118.11) (width 1) (layer "F.Cu") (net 6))
 (segment (start 76.908 91.264) (end 75.208 92.964) (width 0.8) (layer "F.Cu") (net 6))
 (segment (start 145.1 126.718019) (end 143.731981 125.35) (width 1.5) (layer "F.Cu") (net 6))
 (segment (start 75.946 93.194) (end 75.946 106.80537) (width 1.5) (layer "F.Cu") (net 6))
 (segment (start 72.908 92.964) (end 75.208 92.964) (width 1.5) (layer "F.Cu") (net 6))
 (segment (start 66.858 117.094) (end 66.294 116.53) (width 1.5) (layer "F.Cu") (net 6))
 (segment (start 70.848 133.25263) (end 70.848 135.872) (width 1.5) (layer "F.Cu") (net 6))
 (segment (start 129.75 128.822) (end 128.778 129.794) (width 0.8) (layer "F.Cu") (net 6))
 (segment (start 114.4015 136.924) (end 119.2455 132.08) (width 1.5) (layer "F.Cu") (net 6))
 (segment (start 116.83 99.21) (end 116.906296 99.21) (width 1) (layer "F.Cu") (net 6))
 (segment (start 81.93463 114.42537) (end 81.534 114.826) (width 1.5) (layer "F.Cu") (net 6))
 (segment (start 131.572 132.08) (end 128.778 132.08) (width 1.5) (layer "F.Cu") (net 6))
 (segment (start 128 108.08) (end 129.202081 108.08) (width 1) (layer "F.Cu") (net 6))
 (segment (start 143.731981 125.35) (end 139.572 125.35) (width 1.5) (layer "F.Cu") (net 6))
 (segment (start 128.778 129.794) (end 128.778 132.08) (width 0.8) (layer "F.Cu") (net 6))
 (segment (start 114.9 112.35) (end 114.9 115.224) (width 0.8) (layer "F.Cu") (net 6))
 (segment (start 129.75 124.968) (end 129.75 128.822) (width 0.8) (layer "F.Cu") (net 6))
 (segment (start 71.9 136.924) (end 81.534 136.924) (width 1.5) (layer "F.Cu") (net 6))
 (segment (start 81.534 136.924) (end 81.534 114.826) (width 1.5) (layer "F.Cu") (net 6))
 (segment (start 135.89 129.032) (end 135.89 130.302) (width 1.5) (layer "F.Cu") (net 6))
 (segment (start 124.170269 104.367892) (end 127.882377 108.08) (width 1) (layer "F.Cu") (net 6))
 (segment (start 113.792 118.11) (end 116.557 118.11) (width 1) (layer "F.Cu") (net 6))
 (segment (start 74.03937 108.204) (end 72.908 108.204) (width 1.5) (layer "F.Cu") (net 6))
 (segment (start 75.946 130.302) (end 75.946 117.842) (width 1.5) (layer "F.Cu") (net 6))
 (segment (start 70.848 135.872) (end 71.9 136.924) (width 1.5) (layer "F.Cu") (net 6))
 (segment (start 139.572 118.449919) (end 139.572 125.35) (width 1) (layer "F.Cu") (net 6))
 (segment (start 122.713704 118.11) (end 129.571704 124.968) (width 1) (layer "F.Cu") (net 6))
 (segment (start 75.946 117.842) (end 75.198 117.094) (width 1.5) (layer "F.Cu") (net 6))
 (segment (start 134.112 132.08) (end 131.572 132.08) (width 1.5) (layer "F.Cu") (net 6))
 (segment (start 128 118.24) (end 129.75 119.99) (width 0.8) (layer "F.Cu") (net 6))
 (segment (start 107.2 121.8) (end 112.75 116.25) (width 1) (layer "F.Cu") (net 6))
 (segment (start 145.1 132.4) (end 145.1 126.718019) (width 1.5) (layer "F.Cu") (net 6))
 (segment (start 129.75 119.99) (end 129.75 124.968) (width 0.8) (layer "F.Cu") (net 6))
 (segment (start 75.208 92.964) (end 75.438 93.194) (width 1.5) (layer "F.Cu") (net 6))
 (segment (start 75.438 106.80537) (end 74.03937 108.204) (width 1.5) (layer "F.Cu") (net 6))
 (segment (start 72.898 132.334) (end 73.914 132.334) (width 1.5) (layer "F.Cu") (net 6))
 (segment (start 129.571704 124.968) (end 129.75 124.968) (width 1) (layer "F.Cu") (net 6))
 (segment (start 116.906296 99.21) (end 122.064188 104.367892) (width 1) (layer "F.Cu") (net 6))
 (segment (start 135.89 130.302) (end 134.112 132.08) (width 1.5) (layer "F.Cu") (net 6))
 (segment (start 72.898 134.874) (end 74.202428 134.874) (width 1.5) (layer "F.Cu") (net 11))
 (segment (start 116.854 138.924) (end 66.732 138.924) (width 1.5) (layer "F.Cu") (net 11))
 (segment (start 77.946 131.130428) (end 77.946 115.782) (width 1.5) (layer "F.Cu") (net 11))
 (segment (start 77.946 115.782) (end 72.908 110.744) (width 1.5) (layer "F.Cu") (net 11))
 (segment (start 136.58 134.62) (end 131.572 134.62) (width 1.5) (layer "F.Cu") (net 11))
 (segment (start 60.65 118.674) (end 66.294 113.03) (width 1.5) (layer "F.Cu") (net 11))
 (segment (start 66.294 113.03) (end 70.622 113.03) (width 1.5) (layer "F.Cu") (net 11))
 (segment (start 66.732 138.924) (end 60.65 132.842) (width 1.5) (layer "F.Cu") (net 11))
 (segment (start 138.8 132.4) (end 136.58 134.62) (width 1.5) (layer "F.Cu") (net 11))
 (segment (start 70.622 113.03) (end 72.908 110.744) (width 1.5) (layer "F.Cu") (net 11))
 (segment (start 74.202428 134.874) (end 77.946 131.130428) (width 1.5) (layer "F.Cu") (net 11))
 (segment (start 121.158 134.62) (end 116.854 138.924) (width 1.5) (layer "F.Cu") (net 11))
 (segment (start 60.65 132.842) (end 60.65 118.674) (width 1.5) (layer "F.Cu") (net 11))
 (segment (start 131.572 134.62) (end 121.158 134.62) (width 1.5) (layer "F.Cu") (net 11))
 (segment (start 72.898 127.254) (end 67.136 127.254) (width 1.5) (layer "F.Cu") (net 13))
 (segment (start 67.136 127.254) (end 67.056 127.174) (width 1.5) (layer "F.Cu") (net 13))
 (segment (start 87.436478 119.634) (end 85.598 119.634) (width 0.8) (layer "F.Cu") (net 23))
 (segment (start 99.15 114.25) (end 92.820478 114.25) (width 0.8) (layer "F.Cu") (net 23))
 (segment (start 92.820478 114.25) (end 87.436478 119.634) (width 0.8) (layer "F.Cu") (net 23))
 (segment (start 72.898 122.174) (end 67.056 122.174) (width 1.5) (layer "F.Cu") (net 15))
 (segment (start 88.138 117.094) (end 85.598 117.094) (width 0.8) (layer "F.Cu") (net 22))
 (segment (start 99.15 112.25) (end 92.982 112.25) (width 0.8) (layer "F.Cu") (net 22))
 (segment (start 92.982 112.25) (end 88.138 117.094) (width 0.8) (layer "F.Cu") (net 22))
 (segment (start 67.056 129.674) (end 72.778 129.674) (width 1.5) (layer "F.Cu") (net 12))
 (segment (start 72.778 129.674) (end 72.898 129.794) (width 1.5) (layer "F.Cu") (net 12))
 (segment (start 67.056 124.674) (end 72.858 124.674) (width 1.5) (layer "F.Cu") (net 14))
 (segment (start 72.858 124.674) (end 72.898 124.714) (width 1.5) (layer "F.Cu") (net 14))
 (segment (start 72.828 103.044) (end 72.908 103.124) (width 1.5) (layer "F.Cu") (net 31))
 (segment (start 67.056 103.044) (end 72.828 103.044) (width 1.5) (layer "F.Cu") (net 31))
 (segment (start 86.36 92.964) (end 93.63 100.234) (width 0.8) (layer "F.Cu") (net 20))
 (segment (start 93.63 100.234) (end 93.63 106.954164) (width 0.8) (layer "F.Cu") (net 20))
 (segment (start 94.925836 108.25) (end 99.15 108.25) (width 0.8) (layer "F.Cu") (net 20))
 (segment (start 93.63 106.954164) (end 94.925836 108.25) (width 0.8) (layer "F.Cu") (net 20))
 (segment (start 72.908 105.664) (end 67.176 105.664) (width 1.5) (layer "F.Cu") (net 32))
 (segment (start 67.176 105.664) (end 67.056 105.544) (width 1.5) (layer "F.Cu") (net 32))
 (segment (start 91.95 107.112642) (end 91.95 101.094) (width 0.8) (layer "F.Cu") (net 21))
 (segment (start 91.95 101.094) (end 86.36 95.504) (width 0.8) (layer "F.Cu") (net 21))
 (segment (start 99.15 110.25) (end 95.087358 110.25) (width 0.8) (layer "F.Cu") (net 21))
 (segment (start 95.087358 110.25) (end 91.95 107.112642) (width 0.8) (layer "F.Cu") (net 21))
 (segment (start 72.908 98.044) (end 67.056 98.044) (width 1.5) (layer "F.Cu") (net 29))
 (segment (start 72.908 100.584) (end 67.096 100.584) (width 1.5) (layer "F.Cu") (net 30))
 (segment (start 67.096 100.584) (end 67.056 100.544) (width 1.5) (layer "F.Cu") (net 30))
 (segment (start 119.634 113.284) (end 119.888 113.03) (width 1) (layer "F.Cu") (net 25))
 (segment (start 116.102 111.352) (end 118.034 113.284) (width 1) (layer "F.Cu") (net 25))
 (segment (start 112.75 110.25) (end 115 110.25) (width 1) (layer "F.Cu") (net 25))
 (segment (start 119.888 113.03) (end 121.666 113.03) (width 1) (layer "F.Cu") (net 25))
 (segment (start 118.618 113.284) (end 118.618 115.541) (width 1) (layer "F.Cu") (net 25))
 (segment (start 118.034 113.284) (end 118.618 113.284) (width 1) (layer "F.Cu") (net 25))
 (segment (start 115 110.25) (end 116.102 111.352) (width 1) (layer "F.Cu") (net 25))
 (segment (start 118.618 113.284) (end 119.634 113.284) (width 1) (layer "F.Cu") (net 25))
 (segment (start 118.872 108.966) (end 124.95 108.966) (width 0.8) (layer "F.Cu") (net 10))
 (segment (start 118.156 108.25) (end 118.872 108.966) (width 0.8) (layer "F.Cu") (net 10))
 (segment (start 124.95 117.73) (end 128 120.78) (width 0.8) (layer "F.Cu") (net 10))
 (segment (start 118.156 108.25) (end 112.75 108.25) (width 0.8) (layer "F.Cu") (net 10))
 (segment (start 124.95 108.966) (end 124.95 117.73) (width 0.8) (layer "F.Cu") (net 10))
 (segment (start 128 110.62) (end 129.202081 110.62) (width 1) (layer "F.Cu") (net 7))
 (segment (start 131.572 112.989919) (end 131.572 129.54) (width 1) (layer "F.Cu") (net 7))
 (segment (start 129.202081 110.62) (end 131.572 112.989919) (width 1) (layer "F.Cu") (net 7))
 (segment (start 128 115.7) (end 127.923704 115.7) (width 1) (layer "F.Cu") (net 9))
 (segment (start 121.998 106.25) (end 123.414 107.666) (width 0.8) (layer "F.Cu") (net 9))
 (segment (start 126.25 113.95) (end 128 115.7) (width 0.8) (layer "F.Cu") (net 9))
 (segment (start 112.75 106.25) (end 121.998 106.25) (width 0.8) (layer "F.Cu") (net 9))
 (segment (start 123.414 107.666) (end 125.488478 107.666) (width 0.8) (layer "F.Cu") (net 9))
 (segment (start 125.488478 107.666) (end 126.25 108.427522) (width 0.8) (layer "F.Cu") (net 9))
 (segment (start 126.25 108.427522) (end 126.25 113.95) (width 0.8) (layer "F.Cu") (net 9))
 (segment (start 133.226 103) (end 149.826 119.6) (width 1) (layer "F.Cu") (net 4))
 (segment (start 149.826 119.6) (end 150.7 119.6) (width 1) (layer "F.Cu") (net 4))
 (segment (start 128 103) (end 133.226 103) (width 1) (layer "F.Cu") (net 4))
 (segment (start 128 97.92) (end 136.02 97.92) (width 1) (layer "F.Cu") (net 2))
 (segment (start 136.02 97.92) (end 148.6 110.5) (width 1) (layer "F.Cu") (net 2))
 (segment (start 148.6 110.5) (end 150.7 110.5) (width 1) (layer "F.Cu") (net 2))
 (segment (start 128 95.38) (end 138.08 95.38) (width 1) (layer "F.Cu") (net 1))
 (segment (start 138.08 95.38) (end 150.7 108) (width 1) (layer "F.Cu") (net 1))
 (segment (start 134.06 100.46) (end 150.7 117.1) (width 1) (layer "F.Cu") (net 3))
 (segment (start 128 100.46) (end 134.06 100.46) (width 1) (layer "F.Cu") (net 3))
 (segment (start 94.742 98.298) (end 95.83 99.386) (width 0.8) (layer "F.Cu") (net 19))
 (segment (start 95.83 105.75) (end 95.33 106.25) (width 1) (layer "F.Cu") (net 19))
 (segment (start 95.83 99.386) (end 95.83 103.25) (width 0.8) (layer "F.Cu") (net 19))
 (segment (start 95.33 106.25) (end 99.15 106.25) (width 1) (layer "F.Cu") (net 19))
 (segment (start 95.83 103.25) (end 95.83 105.75) (width 1) (layer "F.Cu") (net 19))
 (segment (start 116.33 102.25) (end 116.83 101.75) (width 1) (layer "F.Cu") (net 27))
 (segment (start 112.75 102.25) (end 116.33 102.25) (width 1) (layer "F.Cu") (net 27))
 (segment (start 116.79 104.25) (end 116.83 104.29) (width 1) (layer "F.Cu") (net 26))
 (segment (start 112.75 104.25) (end 116.79 104.25) (width 1) (layer "F.Cu") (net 26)))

